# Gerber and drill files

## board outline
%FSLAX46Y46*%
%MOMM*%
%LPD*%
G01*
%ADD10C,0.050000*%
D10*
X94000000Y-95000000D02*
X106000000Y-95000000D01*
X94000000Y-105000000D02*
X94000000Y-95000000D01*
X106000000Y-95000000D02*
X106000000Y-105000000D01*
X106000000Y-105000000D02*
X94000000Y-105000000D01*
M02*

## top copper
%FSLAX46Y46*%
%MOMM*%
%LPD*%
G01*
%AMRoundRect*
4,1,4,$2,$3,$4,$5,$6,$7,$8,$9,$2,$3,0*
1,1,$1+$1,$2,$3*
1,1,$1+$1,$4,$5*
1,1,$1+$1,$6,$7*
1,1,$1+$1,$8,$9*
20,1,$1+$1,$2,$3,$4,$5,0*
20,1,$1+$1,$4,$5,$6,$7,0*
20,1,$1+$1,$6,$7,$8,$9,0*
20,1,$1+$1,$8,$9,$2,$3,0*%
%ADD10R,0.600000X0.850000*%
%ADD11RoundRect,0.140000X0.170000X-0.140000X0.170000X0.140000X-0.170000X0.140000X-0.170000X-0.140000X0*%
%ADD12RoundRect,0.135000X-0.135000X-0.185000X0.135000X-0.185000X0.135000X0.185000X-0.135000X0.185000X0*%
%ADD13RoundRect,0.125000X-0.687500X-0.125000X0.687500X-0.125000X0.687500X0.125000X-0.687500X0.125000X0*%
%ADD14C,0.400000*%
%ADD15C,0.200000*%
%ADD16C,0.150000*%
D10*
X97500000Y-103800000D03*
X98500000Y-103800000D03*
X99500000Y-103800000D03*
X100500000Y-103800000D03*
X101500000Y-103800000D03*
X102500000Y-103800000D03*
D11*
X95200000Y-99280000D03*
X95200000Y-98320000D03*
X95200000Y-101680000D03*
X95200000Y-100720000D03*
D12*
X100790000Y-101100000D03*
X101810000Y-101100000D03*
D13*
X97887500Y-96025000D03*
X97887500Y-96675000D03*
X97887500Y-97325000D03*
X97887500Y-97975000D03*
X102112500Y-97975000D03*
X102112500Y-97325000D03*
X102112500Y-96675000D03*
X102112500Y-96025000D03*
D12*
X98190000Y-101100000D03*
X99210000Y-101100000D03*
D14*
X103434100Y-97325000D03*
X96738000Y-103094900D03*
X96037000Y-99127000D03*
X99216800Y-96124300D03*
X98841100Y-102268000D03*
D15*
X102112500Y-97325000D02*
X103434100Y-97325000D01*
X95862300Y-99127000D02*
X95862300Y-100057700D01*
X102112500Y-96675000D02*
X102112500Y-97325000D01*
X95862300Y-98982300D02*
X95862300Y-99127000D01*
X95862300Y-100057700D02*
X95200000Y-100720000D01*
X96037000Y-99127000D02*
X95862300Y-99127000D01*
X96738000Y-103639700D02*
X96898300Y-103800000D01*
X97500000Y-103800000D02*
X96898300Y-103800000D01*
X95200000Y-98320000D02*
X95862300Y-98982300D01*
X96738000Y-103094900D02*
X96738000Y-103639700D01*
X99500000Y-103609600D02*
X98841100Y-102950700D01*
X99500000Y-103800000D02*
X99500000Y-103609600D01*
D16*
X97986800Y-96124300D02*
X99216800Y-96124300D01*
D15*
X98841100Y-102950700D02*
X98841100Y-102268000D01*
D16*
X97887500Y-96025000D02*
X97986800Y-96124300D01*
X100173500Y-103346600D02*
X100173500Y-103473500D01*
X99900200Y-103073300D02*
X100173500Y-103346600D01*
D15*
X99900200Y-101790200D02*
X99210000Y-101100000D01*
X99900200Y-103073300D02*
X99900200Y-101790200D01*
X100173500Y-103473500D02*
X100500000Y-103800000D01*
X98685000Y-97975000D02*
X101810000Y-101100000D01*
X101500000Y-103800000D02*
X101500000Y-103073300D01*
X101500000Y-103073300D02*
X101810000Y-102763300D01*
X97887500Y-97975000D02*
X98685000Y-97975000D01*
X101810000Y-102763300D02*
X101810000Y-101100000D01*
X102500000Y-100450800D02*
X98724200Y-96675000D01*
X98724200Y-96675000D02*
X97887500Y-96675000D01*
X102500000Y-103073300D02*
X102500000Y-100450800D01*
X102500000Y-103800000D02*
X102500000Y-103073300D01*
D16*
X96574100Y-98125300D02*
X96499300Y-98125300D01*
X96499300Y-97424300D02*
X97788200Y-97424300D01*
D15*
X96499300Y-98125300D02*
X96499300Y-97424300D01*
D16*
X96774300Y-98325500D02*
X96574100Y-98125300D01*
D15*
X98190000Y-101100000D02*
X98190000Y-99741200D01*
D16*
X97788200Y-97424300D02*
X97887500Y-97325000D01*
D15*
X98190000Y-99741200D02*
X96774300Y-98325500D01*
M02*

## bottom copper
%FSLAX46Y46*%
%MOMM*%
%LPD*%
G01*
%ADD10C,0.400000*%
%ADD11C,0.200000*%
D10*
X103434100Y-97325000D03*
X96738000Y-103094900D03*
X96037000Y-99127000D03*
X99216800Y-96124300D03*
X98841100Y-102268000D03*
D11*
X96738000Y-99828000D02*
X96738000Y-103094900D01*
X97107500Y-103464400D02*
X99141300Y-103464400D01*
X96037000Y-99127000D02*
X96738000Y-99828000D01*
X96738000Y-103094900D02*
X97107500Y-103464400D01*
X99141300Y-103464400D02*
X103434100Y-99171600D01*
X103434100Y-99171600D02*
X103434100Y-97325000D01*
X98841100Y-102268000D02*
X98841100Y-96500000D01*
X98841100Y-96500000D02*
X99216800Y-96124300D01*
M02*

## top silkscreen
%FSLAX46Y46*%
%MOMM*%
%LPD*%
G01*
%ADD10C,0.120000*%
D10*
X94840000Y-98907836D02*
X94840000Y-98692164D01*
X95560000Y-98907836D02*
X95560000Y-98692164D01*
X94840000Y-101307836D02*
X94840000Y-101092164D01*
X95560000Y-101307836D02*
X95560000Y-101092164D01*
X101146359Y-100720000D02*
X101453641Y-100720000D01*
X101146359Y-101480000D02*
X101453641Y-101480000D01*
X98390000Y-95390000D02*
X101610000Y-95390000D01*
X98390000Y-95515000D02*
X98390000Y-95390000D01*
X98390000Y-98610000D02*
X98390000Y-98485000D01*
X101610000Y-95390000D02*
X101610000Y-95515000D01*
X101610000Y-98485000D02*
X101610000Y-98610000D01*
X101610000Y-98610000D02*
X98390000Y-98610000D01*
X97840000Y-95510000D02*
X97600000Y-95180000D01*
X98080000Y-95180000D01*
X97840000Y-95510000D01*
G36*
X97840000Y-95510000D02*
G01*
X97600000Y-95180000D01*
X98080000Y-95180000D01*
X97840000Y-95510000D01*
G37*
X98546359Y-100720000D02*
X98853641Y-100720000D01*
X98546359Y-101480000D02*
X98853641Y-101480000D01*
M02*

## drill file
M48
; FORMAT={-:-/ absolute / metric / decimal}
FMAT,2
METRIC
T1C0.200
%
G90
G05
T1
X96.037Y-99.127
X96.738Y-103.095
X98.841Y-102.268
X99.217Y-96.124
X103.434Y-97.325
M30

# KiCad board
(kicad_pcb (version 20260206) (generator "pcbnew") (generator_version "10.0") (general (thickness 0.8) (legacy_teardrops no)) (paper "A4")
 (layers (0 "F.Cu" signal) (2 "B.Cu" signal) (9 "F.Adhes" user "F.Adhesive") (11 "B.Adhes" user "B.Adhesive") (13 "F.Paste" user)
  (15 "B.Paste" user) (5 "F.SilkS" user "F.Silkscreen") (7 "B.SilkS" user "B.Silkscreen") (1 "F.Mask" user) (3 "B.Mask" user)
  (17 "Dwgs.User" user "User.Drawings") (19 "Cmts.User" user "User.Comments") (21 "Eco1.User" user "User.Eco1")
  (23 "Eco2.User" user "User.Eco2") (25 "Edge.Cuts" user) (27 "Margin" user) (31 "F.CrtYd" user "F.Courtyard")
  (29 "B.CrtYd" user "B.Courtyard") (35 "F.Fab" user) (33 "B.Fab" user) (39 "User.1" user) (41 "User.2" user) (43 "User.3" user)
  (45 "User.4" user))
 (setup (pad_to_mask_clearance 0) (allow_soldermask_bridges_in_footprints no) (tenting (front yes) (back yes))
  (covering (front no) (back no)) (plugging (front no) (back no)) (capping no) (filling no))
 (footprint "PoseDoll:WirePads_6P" (layer "F.Cu") (at 100 103.8)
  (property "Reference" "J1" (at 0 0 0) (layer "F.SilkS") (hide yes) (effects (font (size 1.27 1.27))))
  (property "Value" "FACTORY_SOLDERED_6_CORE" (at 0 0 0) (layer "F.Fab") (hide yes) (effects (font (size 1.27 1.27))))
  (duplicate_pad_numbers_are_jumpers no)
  (pad "1" smd rect (at -2.5 0) (size 0.6 0.85) (layers "F.Cu" "F.Mask") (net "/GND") (thermal_bridge_angle 45))
  (pad "2" smd rect (at -1.5 0) (size 0.6 0.85) (layers "F.Cu" "F.Mask") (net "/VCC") (thermal_bridge_angle 45))
  (pad "3" smd rect (at -0.5 0) (size 0.6 0.85) (layers "F.Cu" "F.Mask") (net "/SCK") (thermal_bridge_angle 45))
  (pad "4" smd rect (at 0.5 0) (size 0.6 0.85) (layers "F.Cu" "F.Mask") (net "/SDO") (thermal_bridge_angle 45))
  (pad "5" smd rect (at 1.5 0) (size 0.6 0.85) (layers "F.Cu" "F.Mask") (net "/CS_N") (thermal_bridge_angle 45))
  (pad "6" smd rect (at 2.5 0) (size 0.6 0.85) (layers "F.Cu" "F.Mask") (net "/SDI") (thermal_bridge_angle 45)))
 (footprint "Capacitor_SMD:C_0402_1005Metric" (layer "F.Cu") (at 95.2 98.8 90)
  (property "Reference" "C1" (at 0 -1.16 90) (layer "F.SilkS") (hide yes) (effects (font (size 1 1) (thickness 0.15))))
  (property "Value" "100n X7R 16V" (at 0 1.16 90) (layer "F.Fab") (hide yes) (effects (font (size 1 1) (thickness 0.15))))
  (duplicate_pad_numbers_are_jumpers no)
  (fp_line (start -0.107836 -0.36) (end 0.107836 -0.36) (stroke (width 0.12) (type solid)) (layer "F.SilkS"))
  (fp_line (start -0.107836 0.36) (end 0.107836 0.36) (stroke (width 0.12) (type solid)) (layer "F.SilkS"))
  (pad "1" smd roundrect (at -0.48 0 90) (size 0.56 0.62) (layers "F.Cu" "F.Mask" "F.Paste") (roundrect_rratio 0.25) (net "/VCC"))
  (pad "2" smd roundrect (at 0.48 0 90) (size 0.56 0.62) (layers "F.Cu" "F.Mask" "F.Paste") (roundrect_rratio 0.25) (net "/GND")))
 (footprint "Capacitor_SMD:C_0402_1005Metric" (layer "F.Cu") (at 95.2 101.2 90)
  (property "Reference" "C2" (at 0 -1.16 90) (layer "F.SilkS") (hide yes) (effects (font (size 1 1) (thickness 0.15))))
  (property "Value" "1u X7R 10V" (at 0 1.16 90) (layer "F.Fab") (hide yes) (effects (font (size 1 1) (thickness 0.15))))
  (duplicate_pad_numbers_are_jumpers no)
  (fp_line (start -0.107836 -0.36) (end 0.107836 -0.36) (stroke (width 0.12) (type solid)) (layer "F.SilkS"))
  (fp_line (start -0.107836 0.36) (end 0.107836 0.36) (stroke (width 0.12) (type solid)) (layer "F.SilkS"))
  (pad "1" smd roundrect (at -0.48 0 90) (size 0.56 0.62) (layers "F.Cu" "F.Mask" "F.Paste") (roundrect_rratio 0.25) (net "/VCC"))
  (pad "2" smd roundrect (at 0.48 0 90) (size 0.56 0.62) (layers "F.Cu" "F.Mask" "F.Paste") (roundrect_rratio 0.25) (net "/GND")))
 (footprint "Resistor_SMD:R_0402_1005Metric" (layer "F.Cu") (at 101.3 101.1)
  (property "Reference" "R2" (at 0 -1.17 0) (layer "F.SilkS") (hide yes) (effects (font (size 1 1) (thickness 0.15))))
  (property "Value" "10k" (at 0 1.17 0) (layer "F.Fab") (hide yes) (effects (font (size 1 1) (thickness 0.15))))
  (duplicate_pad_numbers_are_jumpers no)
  (fp_line (start -0.153641 -0.38) (end 0.153641 -0.38) (stroke (width 0.12) (type solid)) (layer "F.SilkS"))
  (fp_line (start -0.153641 0.38) (end 0.153641 0.38) (stroke (width 0.12) (type solid)) (layer "F.SilkS"))
  (pad "1" smd roundrect (at -0.51 0) (size 0.54 0.64) (layers "F.Cu" "F.Mask" "F.Paste") (roundrect_rratio 0.25) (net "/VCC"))
  (pad "2" smd roundrect (at 0.51 0) (size 0.54 0.64) (layers "F.Cu" "F.Mask" "F.Paste") (roundrect_rratio 0.25) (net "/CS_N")))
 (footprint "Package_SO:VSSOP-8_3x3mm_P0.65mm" (layer "F.Cu") (at 100 97)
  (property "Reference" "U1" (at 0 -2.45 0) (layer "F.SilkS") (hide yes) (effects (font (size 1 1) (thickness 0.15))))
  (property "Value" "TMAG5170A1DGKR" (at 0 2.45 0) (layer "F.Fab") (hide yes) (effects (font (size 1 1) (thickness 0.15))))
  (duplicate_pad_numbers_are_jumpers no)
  (fp_line (start -1.61 -1.61) (end 1.61 -1.61) (stroke (width 0.12) (type solid)) (layer "F.SilkS"))
  (fp_line (start -1.61 -1.485) (end -1.61 -1.61) (stroke (width 0.12) (type solid)) (layer "F.SilkS"))
  (fp_line (start -1.61 1.61) (end -1.61 1.485) (stroke (width 0.12) (type solid)) (layer "F.SilkS"))
  (fp_line (start 1.61 -1.61) (end 1.61 -1.485) (stroke (width 0.12) (type solid)) (layer "F.SilkS"))
  (fp_line (start 1.61 1.485) (end 1.61 1.61) (stroke (width 0.12) (type solid)) (layer "F.SilkS"))
  (fp_line (start 1.61 1.61) (end -1.61 1.61) (stroke (width 0.12) (type solid)) (layer "F.SilkS"))
  (fp_poly (pts (xy -2.16 -1.49) (xy -2.4 -1.82) (xy -1.92 -1.82)) (stroke (width 0.12) (type solid)) (fill yes) (layer "F.SilkS"))
  (pad "1" smd roundrect (at -2.1125 -0.975) (size 1.625 0.5) (layers "F.Cu" "F.Mask" "F.Paste") (roundrect_rratio 0.25) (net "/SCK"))
  (pad "2" smd roundrect (at -2.1125 -0.325) (size 1.625 0.5) (layers "F.Cu" "F.Mask" "F.Paste") (roundrect_rratio 0.25) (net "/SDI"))
  (pad "3" smd roundrect (at -2.1125 0.325) (size 1.625 0.5) (layers "F.Cu" "F.Mask" "F.Paste") (roundrect_rratio 0.25) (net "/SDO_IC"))
  (pad "4" smd roundrect (at -2.1125 0.975) (size 1.625 0.5) (layers "F.Cu" "F.Mask" "F.Paste") (roundrect_rratio 0.25) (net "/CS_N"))
  (pad "5" smd roundrect (at 2.1125 0.975) (size 1.625 0.5) (layers "F.Cu" "F.Mask" "F.Paste") (roundrect_rratio 0.25) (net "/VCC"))
  (pad "6" smd roundrect (at 2.1125 0.325) (size 1.625 0.5) (layers "F.Cu" "F.Mask" "F.Paste") (roundrect_rratio 0.25) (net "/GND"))
  (pad "7" smd roundrect (at 2.1125 -0.325) (size 1.625 0.5) (layers "F.Cu" "F.Mask" "F.Paste") (roundrect_rratio 0.25) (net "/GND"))
  (pad "8" smd roundrect (at 2.1125 -0.975) (size 1.625 0.5) (layers "F.Cu" "F.Mask" "F.Paste") (roundrect_rratio 0.25)
   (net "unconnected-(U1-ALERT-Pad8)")))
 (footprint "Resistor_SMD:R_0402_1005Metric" (layer "F.Cu") (at 98.7 101.1)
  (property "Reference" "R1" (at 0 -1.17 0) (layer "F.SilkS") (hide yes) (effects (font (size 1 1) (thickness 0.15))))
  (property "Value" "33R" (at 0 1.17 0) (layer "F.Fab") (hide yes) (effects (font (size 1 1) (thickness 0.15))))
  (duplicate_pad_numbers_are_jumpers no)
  (fp_line (start -0.153641 -0.38) (end 0.153641 -0.38) (stroke (width 0.12) (type solid)) (layer "F.SilkS"))
  (fp_line (start -0.153641 0.38) (end 0.153641 0.38) (stroke (width 0.12) (type solid)) (layer "F.SilkS"))
  (pad "1" smd roundrect (at -0.51 0) (size 0.54 0.64) (layers "F.Cu" "F.Mask" "F.Paste") (roundrect_rratio 0.25) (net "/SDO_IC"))
  (pad "2" smd roundrect (at 0.51 0) (size 0.54 0.64) (layers "F.Cu" "F.Mask" "F.Paste") (roundrect_rratio 0.25) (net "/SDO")))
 (gr_line (start 94 95) (end 106 95) (stroke (width 0.05) (type default)) (layer "Edge.Cuts"))
 (gr_line (start 94 105) (end 94 95) (stroke (width 0.05) (type default)) (layer "Edge.Cuts"))
 (gr_line (start 106 95) (end 106 105) (stroke (width 0.05) (type default)) (layer "Edge.Cuts"))
 (gr_line (start 106 105) (end 94 105) (stroke (width 0.05) (type default)) (layer "Edge.Cuts"))
 (segment (start 102.1125 97.325) (end 103.4341 97.325) (width 0.2) (layer "F.Cu") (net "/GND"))
 (segment (start 95.8623 99.127) (end 95.8623 100.0577) (width 0.2) (layer "F.Cu") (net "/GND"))
 (segment (start 102.1125 96.675) (end 102.1125 97.325) (width 0.2) (layer "F.Cu") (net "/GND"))
 (segment (start 95.8623 98.9823) (end 95.8623 99.127) (width 0.2) (layer "F.Cu") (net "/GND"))
 (segment (start 95.8623 100.0577) (end 95.2 100.72) (width 0.2) (layer "F.Cu") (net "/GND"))
 (segment (start 96.037 99.127) (end 95.8623 99.127) (width 0.2) (layer "F.Cu") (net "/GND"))
 (segment (start 96.738 103.6397) (end 96.8983 103.8) (width 0.2) (layer "F.Cu") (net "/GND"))
 (segment (start 97.5 103.8) (end 96.8983 103.8) (width 0.2) (layer "F.Cu") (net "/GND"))
 (segment (start 95.2 98.32) (end 95.8623 98.9823) (width 0.2) (layer "F.Cu") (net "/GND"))
 (segment (start 96.738 103.0949) (end 96.738 103.6397) (width 0.2) (layer "F.Cu") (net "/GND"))
 (via (at 103.4341 97.325) (size 0.4) (drill 0.2) (layers "F.Cu" "B.Cu") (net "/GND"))
 (via (at 96.738 103.0949) (size 0.4) (drill 0.2) (layers "F.Cu" "B.Cu") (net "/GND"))
 (via (at 96.037 99.127) (size 0.4) (drill 0.2) (layers "F.Cu" "B.Cu") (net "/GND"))
 (segment (start 96.738 99.828) (end 96.738 103.0949) (width 0.2) (layer "B.Cu") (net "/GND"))
 (segment (start 97.1075 103.4644) (end 99.1413 103.4644) (width 0.2) (layer "B.Cu") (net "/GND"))
 (segment (start 96.037 99.127) (end 96.738 99.828) (width 0.2) (layer "B.Cu") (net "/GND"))
 (segment (start 96.738 103.0949) (end 97.1075 103.4644) (width 0.2) (layer "B.Cu") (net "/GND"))
 (segment (start 99.1413 103.4644) (end 103.4341 99.1716) (width 0.2) (layer "B.Cu") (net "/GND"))
 (segment (start 103.4341 99.1716) (end 103.4341 97.325) (width 0.2) (layer "B.Cu") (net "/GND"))
 (segment (start 99.5 103.6096) (end 98.8411 102.9507) (width 0.2) (layer "F.Cu") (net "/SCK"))
 (segment (start 99.5 103.8) (end 99.5 103.6096) (width 0.2) (layer "F.Cu") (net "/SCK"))
 (segment (start 97.9868 96.1243) (end 99.2168 96.1243) (width 0.15) (layer "F.Cu") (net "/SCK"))
 (segment (start 98.8411 102.9507) (end 98.8411 102.268) (width 0.2) (layer "F.Cu") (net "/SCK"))
 (segment (start 97.8875 96.025) (end 97.9868 96.1243) (width 0.15) (layer "F.Cu") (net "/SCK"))
 (via (at 99.2168 96.1243) (size 0.4) (drill 0.2) (layers "F.Cu" "B.Cu") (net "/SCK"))
 (via (at 98.8411 102.268) (size 0.4) (drill 0.2) (layers "F.Cu" "B.Cu") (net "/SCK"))
 (segment (start 98.8411 102.268) (end 98.8411 96.5) (width 0.2) (layer "B.Cu") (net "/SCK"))
 (segment (start 98.8411 96.5) (end 99.2168 96.1243) (width 0.2) (layer "B.Cu") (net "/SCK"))
 (segment (start 100.1735 103.3466) (end 100.1735 103.4735) (width 0.15) (layer "F.Cu") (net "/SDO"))
 (segment (start 99.9002 103.0733) (end 100.1735 103.3466) (width 0.15) (layer "F.Cu") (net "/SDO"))
 (segment (start 99.9002 101.7902) (end 99.21 101.1) (width 0.2) (layer "F.Cu") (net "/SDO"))
 (segment (start 99.9002 103.0733) (end 99.9002 101.7902) (width 0.2) (layer "F.Cu") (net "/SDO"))
 (segment (start 100.1735 103.4735) (end 100.5 103.8) (width 0.2) (layer "F.Cu") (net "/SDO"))
 (segment (start 98.685 97.975) (end 101.81 101.1) (width 0.2) (layer "F.Cu") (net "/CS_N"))
 (segment (start 101.5 103.8) (end 101.5 103.0733) (width 0.2) (layer "F.Cu") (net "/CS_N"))
 (segment (start 101.5 103.0733) (end 101.81 102.7633) (width 0.2) (layer "F.Cu") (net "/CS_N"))
 (segment (start 97.8875 97.975) (end 98.685 97.975) (width 0.2) (layer "F.Cu") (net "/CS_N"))
 (segment (start 101.81 102.7633) (end 101.81 101.1) (width 0.2) (layer "F.Cu") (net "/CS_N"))
 (segment (start 102.5 100.4508) (end 98.7242 96.675) (width 0.2) (layer "F.Cu") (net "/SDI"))
 (segment (start 98.7242 96.675) (end 97.8875 96.675) (width 0.2) (layer "F.Cu") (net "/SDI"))
 (segment (start 102.5 103.0733) (end 102.5 100.4508) (width 0.2) (layer "F.Cu") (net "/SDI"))
 (segment (start 102.5 103.8) (end 102.5 103.0733) (width 0.2) (layer "F.Cu") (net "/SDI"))
 (segment (start 96.5741 98.1253) (end 96.4993 98.1253) (width 0.15) (layer "F.Cu") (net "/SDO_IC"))
 (segment (start 96.4993 97.4243) (end 97.7882 97.4243) (width 0.15) (layer "F.Cu") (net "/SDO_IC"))
 (segment (start 96.4993 98.1253) (end 96.4993 97.4243) (width 0.2) (layer "F.Cu") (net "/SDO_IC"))
 (segment (start 96.7743 98.3255) (end 96.5741 98.1253) (width 0.15) (layer "F.Cu") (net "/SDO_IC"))
 (segment (start 98.19 101.1) (end 98.19 99.7412) (width 0.2) (layer "F.Cu") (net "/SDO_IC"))
 (segment (start 97.7882 97.4243) (end 97.8875 97.325) (width 0.15) (layer "F.Cu") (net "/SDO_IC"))
 (segment (start 98.19 99.7412) (end 96.7743 98.3255) (width 0.2) (layer "F.Cu") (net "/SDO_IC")))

